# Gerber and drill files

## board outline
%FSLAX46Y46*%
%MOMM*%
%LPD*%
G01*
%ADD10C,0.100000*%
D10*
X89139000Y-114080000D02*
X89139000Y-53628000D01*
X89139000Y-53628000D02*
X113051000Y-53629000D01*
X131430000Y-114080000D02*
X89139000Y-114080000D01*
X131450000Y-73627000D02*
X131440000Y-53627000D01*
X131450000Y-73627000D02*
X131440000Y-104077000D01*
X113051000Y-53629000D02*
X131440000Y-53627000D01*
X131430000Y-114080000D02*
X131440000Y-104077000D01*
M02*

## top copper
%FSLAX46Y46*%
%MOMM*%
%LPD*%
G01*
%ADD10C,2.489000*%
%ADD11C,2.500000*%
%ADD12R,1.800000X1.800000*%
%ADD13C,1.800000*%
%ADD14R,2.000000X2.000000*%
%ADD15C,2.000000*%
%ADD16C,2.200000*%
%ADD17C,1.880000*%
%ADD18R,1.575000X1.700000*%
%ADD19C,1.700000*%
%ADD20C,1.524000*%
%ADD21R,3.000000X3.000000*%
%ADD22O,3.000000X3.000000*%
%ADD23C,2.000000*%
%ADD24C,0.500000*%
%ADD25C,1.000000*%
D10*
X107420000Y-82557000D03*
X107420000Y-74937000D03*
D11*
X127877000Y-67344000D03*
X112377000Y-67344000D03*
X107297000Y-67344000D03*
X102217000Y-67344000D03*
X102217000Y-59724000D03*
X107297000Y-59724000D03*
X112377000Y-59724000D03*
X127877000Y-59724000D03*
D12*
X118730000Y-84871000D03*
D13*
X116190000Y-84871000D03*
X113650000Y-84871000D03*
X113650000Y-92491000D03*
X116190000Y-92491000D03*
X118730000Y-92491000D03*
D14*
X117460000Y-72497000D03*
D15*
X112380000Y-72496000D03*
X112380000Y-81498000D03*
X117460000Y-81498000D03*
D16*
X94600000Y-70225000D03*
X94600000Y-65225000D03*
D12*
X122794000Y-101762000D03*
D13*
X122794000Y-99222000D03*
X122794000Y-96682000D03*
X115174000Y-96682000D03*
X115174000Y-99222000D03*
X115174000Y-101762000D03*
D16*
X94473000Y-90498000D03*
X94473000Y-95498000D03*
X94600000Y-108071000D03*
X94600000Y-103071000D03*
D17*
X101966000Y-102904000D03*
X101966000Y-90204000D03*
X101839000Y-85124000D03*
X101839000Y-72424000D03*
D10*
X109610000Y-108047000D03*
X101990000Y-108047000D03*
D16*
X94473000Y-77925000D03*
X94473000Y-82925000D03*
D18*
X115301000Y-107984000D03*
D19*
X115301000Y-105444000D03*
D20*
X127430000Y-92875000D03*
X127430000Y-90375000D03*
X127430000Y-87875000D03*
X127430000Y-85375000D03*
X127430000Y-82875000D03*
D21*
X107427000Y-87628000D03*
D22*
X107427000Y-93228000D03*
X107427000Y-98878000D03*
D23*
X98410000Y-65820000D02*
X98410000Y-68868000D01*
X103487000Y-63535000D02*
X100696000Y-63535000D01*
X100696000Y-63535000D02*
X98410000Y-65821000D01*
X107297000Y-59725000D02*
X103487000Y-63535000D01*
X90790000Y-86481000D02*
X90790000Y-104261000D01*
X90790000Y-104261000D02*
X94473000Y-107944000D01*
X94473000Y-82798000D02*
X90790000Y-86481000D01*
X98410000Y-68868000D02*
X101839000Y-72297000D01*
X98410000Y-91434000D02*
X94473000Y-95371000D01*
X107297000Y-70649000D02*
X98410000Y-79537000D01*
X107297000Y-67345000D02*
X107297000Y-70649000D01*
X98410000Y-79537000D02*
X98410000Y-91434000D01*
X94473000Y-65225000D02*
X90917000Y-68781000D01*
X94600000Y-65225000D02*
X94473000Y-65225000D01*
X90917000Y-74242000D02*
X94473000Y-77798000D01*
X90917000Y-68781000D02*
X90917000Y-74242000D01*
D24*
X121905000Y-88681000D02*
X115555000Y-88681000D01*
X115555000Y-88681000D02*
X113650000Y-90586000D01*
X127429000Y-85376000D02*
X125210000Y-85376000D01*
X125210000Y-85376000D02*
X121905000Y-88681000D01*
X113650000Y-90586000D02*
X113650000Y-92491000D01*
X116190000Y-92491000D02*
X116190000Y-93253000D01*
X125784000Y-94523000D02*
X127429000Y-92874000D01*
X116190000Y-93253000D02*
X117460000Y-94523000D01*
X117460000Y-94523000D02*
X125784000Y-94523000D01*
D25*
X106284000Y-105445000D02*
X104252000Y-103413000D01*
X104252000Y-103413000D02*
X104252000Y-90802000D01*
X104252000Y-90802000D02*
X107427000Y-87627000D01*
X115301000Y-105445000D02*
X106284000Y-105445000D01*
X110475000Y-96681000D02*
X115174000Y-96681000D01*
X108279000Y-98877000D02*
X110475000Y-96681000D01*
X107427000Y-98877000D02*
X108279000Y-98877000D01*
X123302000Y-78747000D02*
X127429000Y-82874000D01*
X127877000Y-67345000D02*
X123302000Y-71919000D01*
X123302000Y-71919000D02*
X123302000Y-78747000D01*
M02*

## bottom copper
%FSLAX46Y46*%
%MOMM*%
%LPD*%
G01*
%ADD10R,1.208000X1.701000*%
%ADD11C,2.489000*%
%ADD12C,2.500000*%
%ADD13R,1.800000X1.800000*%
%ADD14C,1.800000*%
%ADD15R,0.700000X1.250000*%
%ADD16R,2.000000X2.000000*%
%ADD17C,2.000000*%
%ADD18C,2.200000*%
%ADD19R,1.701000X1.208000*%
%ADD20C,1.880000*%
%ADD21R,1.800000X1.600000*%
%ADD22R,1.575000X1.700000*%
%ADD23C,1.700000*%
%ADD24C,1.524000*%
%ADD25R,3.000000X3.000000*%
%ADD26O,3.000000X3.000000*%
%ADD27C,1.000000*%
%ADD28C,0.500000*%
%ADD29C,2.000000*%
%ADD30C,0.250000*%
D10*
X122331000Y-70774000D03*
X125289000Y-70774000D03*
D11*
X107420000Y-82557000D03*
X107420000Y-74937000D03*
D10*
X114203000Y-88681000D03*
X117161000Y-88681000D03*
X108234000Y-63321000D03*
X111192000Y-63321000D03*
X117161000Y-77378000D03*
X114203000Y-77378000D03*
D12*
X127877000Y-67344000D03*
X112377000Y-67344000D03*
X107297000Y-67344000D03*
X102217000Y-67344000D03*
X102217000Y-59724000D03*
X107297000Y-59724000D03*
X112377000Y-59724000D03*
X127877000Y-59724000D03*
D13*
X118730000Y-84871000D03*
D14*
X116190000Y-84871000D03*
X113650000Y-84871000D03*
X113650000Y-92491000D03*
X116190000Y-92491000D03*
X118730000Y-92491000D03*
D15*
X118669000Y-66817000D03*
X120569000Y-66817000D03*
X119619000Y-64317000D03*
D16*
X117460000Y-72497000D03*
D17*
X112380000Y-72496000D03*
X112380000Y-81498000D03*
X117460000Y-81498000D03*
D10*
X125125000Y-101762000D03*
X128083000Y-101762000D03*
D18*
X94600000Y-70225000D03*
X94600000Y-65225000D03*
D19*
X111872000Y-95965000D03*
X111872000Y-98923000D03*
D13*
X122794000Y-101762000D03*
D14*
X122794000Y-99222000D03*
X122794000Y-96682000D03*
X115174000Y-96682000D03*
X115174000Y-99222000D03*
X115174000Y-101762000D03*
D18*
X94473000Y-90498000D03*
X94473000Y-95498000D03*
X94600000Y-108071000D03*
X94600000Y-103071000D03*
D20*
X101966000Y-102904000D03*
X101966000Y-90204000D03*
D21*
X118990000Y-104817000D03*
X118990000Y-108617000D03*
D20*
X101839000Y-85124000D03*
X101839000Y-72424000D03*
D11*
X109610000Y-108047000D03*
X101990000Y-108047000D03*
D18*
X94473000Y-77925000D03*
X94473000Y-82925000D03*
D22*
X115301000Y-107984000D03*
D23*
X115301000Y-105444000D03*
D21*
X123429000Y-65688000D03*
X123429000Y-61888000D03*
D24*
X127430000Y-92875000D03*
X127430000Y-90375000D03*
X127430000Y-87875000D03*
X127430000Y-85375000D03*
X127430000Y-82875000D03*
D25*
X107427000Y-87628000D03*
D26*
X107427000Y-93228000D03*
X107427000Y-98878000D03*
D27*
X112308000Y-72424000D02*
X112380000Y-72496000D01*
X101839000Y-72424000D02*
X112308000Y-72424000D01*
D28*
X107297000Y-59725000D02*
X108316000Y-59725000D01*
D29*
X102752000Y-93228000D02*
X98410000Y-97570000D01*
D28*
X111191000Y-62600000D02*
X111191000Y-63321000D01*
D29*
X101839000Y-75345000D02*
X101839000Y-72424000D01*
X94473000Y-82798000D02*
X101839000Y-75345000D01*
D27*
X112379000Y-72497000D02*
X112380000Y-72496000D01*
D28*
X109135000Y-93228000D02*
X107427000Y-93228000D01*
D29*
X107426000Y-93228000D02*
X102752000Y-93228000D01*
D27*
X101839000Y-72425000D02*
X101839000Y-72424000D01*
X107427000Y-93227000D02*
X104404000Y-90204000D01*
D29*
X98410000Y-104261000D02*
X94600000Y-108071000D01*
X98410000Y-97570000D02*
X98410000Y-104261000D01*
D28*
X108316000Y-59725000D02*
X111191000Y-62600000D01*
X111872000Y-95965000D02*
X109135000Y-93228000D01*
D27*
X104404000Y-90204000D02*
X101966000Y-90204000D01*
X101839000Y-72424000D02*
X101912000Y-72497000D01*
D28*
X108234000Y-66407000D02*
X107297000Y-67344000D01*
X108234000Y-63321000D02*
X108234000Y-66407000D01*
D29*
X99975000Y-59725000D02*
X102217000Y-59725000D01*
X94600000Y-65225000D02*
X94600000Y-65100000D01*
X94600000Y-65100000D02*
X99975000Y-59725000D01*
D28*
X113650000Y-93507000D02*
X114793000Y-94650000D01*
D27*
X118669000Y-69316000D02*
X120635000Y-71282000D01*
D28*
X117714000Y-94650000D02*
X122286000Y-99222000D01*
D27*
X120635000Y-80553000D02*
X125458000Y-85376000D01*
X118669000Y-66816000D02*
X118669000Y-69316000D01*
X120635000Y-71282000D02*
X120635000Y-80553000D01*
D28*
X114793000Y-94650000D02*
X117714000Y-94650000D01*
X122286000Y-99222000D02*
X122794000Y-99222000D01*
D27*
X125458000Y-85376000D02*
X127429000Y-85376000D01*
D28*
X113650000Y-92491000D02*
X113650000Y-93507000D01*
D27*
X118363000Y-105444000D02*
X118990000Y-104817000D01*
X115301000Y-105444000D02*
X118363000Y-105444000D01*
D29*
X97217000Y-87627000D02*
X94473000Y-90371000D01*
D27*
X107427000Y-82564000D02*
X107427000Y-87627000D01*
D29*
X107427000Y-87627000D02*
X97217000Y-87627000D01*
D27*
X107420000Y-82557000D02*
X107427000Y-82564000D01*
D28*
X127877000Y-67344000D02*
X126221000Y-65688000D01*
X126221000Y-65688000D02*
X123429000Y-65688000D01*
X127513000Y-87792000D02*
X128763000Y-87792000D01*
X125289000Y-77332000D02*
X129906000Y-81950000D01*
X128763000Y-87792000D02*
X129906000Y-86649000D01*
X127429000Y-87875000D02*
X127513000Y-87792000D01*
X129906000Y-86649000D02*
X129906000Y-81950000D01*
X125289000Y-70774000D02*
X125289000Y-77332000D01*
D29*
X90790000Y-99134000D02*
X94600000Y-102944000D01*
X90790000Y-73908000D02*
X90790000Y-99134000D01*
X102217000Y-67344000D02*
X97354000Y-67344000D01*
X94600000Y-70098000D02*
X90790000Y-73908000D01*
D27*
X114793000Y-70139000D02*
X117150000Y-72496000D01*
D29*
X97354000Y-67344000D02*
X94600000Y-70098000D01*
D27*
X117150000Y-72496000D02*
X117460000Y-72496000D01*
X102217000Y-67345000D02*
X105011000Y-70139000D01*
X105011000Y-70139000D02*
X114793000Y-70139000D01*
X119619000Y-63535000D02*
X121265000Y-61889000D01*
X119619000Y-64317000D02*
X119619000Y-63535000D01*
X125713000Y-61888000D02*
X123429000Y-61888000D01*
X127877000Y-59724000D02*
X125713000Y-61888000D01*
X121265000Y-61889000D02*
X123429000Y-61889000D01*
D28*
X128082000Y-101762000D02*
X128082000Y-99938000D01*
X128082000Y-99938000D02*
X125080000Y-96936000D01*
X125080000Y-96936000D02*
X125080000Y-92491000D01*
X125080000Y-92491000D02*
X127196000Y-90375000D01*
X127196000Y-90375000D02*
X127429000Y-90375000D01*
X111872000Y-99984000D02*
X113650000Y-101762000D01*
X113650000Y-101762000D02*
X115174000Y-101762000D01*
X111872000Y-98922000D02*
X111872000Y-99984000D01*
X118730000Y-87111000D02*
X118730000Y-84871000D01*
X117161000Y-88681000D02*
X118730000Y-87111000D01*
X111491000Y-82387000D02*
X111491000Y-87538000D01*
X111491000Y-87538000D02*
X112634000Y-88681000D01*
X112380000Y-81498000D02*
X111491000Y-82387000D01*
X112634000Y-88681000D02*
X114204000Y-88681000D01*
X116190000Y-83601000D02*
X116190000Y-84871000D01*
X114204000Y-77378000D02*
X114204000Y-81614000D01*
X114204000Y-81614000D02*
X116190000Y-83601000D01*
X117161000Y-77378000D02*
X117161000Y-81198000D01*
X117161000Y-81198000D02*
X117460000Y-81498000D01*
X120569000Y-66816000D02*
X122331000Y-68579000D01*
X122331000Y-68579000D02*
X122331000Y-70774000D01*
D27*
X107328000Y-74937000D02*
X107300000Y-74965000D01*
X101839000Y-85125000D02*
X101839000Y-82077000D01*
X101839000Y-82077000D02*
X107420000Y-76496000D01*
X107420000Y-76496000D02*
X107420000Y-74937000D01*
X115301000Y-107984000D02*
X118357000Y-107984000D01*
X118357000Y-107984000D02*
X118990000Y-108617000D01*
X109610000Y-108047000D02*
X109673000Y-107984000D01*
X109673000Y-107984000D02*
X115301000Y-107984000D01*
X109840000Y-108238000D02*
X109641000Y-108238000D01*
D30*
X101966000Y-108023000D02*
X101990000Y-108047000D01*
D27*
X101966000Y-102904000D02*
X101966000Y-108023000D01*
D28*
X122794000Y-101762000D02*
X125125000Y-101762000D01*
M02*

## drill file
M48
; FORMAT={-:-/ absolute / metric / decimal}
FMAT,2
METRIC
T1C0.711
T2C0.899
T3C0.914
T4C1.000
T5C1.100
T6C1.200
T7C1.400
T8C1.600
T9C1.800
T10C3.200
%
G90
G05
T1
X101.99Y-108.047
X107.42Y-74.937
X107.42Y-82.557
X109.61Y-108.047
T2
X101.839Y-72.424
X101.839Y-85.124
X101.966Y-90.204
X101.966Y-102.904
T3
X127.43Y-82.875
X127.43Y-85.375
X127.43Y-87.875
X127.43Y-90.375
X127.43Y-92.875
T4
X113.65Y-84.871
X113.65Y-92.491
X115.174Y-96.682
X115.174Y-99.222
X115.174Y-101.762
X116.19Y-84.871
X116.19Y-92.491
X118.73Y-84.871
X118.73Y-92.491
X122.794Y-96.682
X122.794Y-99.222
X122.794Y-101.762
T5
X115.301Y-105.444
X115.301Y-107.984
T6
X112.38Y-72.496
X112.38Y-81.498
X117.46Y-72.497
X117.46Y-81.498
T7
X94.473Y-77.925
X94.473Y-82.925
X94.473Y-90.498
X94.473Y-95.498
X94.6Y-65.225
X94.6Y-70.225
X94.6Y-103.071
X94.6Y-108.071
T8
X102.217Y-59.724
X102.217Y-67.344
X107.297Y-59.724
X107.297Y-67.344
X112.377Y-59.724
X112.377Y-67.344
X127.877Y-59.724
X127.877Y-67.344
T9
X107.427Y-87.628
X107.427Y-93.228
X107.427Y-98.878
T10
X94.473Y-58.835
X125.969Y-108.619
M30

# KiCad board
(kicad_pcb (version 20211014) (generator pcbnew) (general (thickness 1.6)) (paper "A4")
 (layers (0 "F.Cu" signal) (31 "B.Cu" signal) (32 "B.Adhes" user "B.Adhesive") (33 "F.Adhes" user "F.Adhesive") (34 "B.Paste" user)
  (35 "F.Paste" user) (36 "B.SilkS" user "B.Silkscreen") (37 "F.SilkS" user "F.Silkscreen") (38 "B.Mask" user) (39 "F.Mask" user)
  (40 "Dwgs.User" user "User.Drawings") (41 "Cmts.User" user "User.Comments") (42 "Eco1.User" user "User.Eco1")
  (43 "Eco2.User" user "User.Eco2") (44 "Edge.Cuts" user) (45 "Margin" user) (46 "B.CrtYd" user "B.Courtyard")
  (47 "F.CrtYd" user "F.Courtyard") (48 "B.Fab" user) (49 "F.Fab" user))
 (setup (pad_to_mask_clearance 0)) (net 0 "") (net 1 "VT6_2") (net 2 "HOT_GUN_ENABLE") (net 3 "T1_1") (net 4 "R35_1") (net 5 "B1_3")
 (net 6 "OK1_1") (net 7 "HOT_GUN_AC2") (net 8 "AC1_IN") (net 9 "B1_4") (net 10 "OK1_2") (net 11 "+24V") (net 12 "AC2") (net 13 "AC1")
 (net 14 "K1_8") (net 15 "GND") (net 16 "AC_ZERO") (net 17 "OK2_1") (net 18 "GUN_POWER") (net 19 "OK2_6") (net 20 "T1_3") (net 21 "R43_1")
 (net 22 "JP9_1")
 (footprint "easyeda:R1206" (layer "F.Cu") (at 123.81 70.774 180)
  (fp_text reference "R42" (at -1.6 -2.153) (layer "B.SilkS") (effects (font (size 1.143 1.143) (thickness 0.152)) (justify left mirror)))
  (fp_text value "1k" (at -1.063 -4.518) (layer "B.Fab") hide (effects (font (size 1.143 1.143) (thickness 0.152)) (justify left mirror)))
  (pad "1" smd rect locked (at 1.479 0 180) (size 1.208 1.701) (layers "B.Cu" "B.Paste" "B.Mask") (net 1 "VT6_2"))
  (pad "2" smd rect locked (at -1.479 0 180) (size 1.208 1.701) (layers "B.Cu" "B.Paste" "B.Mask") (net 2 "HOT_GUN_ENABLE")))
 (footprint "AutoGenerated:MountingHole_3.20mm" (layer "F.Cu") (at 125.969 108.619)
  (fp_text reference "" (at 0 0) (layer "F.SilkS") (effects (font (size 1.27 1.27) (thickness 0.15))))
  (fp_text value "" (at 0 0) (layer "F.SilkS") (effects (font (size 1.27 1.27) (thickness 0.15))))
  (pad "" np_thru_hole circle locked (at 0 0) (size 3.2 3.2) (drill 3.2) (layers *.Cu *.Mask)))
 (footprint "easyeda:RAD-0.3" (layer "F.Cu") (at 107.42 78.747 -90)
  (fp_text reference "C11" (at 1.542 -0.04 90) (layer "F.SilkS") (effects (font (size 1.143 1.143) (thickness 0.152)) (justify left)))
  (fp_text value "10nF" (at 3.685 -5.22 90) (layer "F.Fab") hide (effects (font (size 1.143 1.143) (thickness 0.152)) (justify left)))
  (pad "1" thru_hole circle locked (at 3.81 0 90) (size 2.489 2.489) (drill 0.711) (layers *.Cu *.Paste *.Mask) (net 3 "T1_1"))
  (pad "2" thru_hole circle locked (at -3.81 0 90) (size 2.489 2.489) (drill 0.711) (layers *.Cu *.Paste *.Mask) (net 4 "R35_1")))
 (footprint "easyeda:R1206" (layer "F.Cu") (at 115.682 88.681 180)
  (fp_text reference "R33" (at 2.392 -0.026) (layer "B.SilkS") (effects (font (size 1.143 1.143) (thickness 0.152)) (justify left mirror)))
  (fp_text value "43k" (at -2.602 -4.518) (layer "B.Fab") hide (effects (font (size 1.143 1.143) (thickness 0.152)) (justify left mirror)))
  (pad "1" smd rect locked (at 1.479 0 180) (size 1.208 1.701) (layers "B.Cu" "B.Paste" "B.Mask") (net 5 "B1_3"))
  (pad "2" smd rect locked (at -1.479 0 180) (size 1.208 1.701) (layers "B.Cu" "B.Paste" "B.Mask") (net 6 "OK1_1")))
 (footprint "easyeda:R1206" (layer "F.Cu") (at 109.713 63.321 180)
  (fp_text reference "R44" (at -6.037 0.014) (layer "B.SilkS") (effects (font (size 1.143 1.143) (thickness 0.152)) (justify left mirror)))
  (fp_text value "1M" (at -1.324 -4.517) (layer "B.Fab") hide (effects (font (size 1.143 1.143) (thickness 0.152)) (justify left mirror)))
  (pad "1" smd rect locked (at 1.479 0 180) (size 1.208 1.701) (layers "B.Cu" "B.Paste" "B.Mask") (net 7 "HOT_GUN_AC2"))
  (pad "2" smd rect locked (at -1.479 0 180) (size 1.208 1.701) (layers "B.Cu" "B.Paste" "B.Mask") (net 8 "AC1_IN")))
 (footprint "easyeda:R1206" (layer "F.Cu") (at 115.682 77.378)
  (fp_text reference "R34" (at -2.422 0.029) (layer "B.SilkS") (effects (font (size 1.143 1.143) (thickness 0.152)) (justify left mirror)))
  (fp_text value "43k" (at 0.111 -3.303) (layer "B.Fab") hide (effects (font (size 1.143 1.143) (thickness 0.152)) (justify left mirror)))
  (pad "1" smd rect locked (at 1.479 0) (size 1.208 1.701) (layers "B.Cu" "B.Paste" "B.Mask") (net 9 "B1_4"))
  (pad "2" smd rect locked (at -1.479 0) (size 1.208 1.701) (layers "B.Cu" "B.Paste" "B.Mask") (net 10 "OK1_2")))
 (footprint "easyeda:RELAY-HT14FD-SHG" (layer "F.Cu") (at 115.047 63.534 180)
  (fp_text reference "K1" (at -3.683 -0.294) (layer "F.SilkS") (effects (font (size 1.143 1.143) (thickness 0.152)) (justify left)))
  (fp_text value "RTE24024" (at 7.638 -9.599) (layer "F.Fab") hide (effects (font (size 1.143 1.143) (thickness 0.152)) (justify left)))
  (pad "1" thru_hole circle locked (at -12.83 -3.81 180) (size 2.5 2.5) (drill 1.6) (layers *.Cu *.Paste *.Mask) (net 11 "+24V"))
  (pad "2" thru_hole circle locked (at 2.67 -3.81 180) (size 2.5 2.5) (drill 1.6) (layers *.Cu *.Paste *.Mask))
  (pad "3" thru_hole circle locked (at 7.75 -3.81 180) (size 2.5 2.5) (drill 1.6) (layers *.Cu *.Paste *.Mask) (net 7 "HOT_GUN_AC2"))
  (pad "4" thru_hole circle locked (at 12.83 -3.81 180) (size 2.5 2.5) (drill 1.6) (layers *.Cu *.Paste *.Mask) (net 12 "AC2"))
  (pad "5" thru_hole circle locked (at 12.83 3.81 180) (size 2.5 2.5) (drill 1.6) (layers *.Cu *.Paste *.Mask) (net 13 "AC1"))
  (pad "6" thru_hole circle locked (at 7.75 3.81 180) (size 2.5 2.5) (drill 1.6) (layers *.Cu *.Paste *.Mask) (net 8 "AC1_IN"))
  (pad "7" thru_hole circle locked (at 2.67 3.81 180) (size 2.5 2.5) (drill 1.6) (layers *.Cu *.Paste *.Mask))
  (pad "8" thru_hole circle locked (at -12.83 3.81 180) (size 2.5 2.5) (drill 1.6) (layers *.Cu *.Paste *.Mask) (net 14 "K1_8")))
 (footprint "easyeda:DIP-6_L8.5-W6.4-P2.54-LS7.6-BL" (layer "F.Cu") (at 116.19 88.681 180)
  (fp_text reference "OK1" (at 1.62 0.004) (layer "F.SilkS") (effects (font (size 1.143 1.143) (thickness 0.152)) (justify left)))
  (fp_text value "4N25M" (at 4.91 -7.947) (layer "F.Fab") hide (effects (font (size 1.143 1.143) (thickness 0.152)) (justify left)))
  (pad "1" thru_hole rect locked (at -2.54 3.81 270) (size 1.8 1.8) (drill 1) (layers *.Cu *.Paste *.Mask) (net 6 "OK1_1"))
  (pad "2" thru_hole circle locked (at 0 3.81 270) (size 1.8 1.8) (drill 1) (layers *.Cu *.Paste *.Mask) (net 10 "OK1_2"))
  (pad "3" thru_hole circle locked (at 2.54 3.81 270) (size 1.8 1.8) (drill 1) (layers *.Cu *.Paste *.Mask))
  (pad "4" thru_hole circle locked (at 2.54 -3.81 270) (size 1.8 1.8) (drill 1) (layers *.Cu *.Paste *.Mask) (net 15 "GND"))
  (pad "5" thru_hole circle locked (at 0 -3.81 270) (size 1.8 1.8) (drill 1) (layers *.Cu *.Paste *.Mask) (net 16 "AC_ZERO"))
  (pad "6" thru_hole circle locked (at -2.54 -3.81 270) (size 1.8 1.8) (drill 1) (layers *.Cu *.Paste *.Mask)))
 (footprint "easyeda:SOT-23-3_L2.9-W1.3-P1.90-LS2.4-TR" (layer "F.Cu") (at 119.619 65.567 90)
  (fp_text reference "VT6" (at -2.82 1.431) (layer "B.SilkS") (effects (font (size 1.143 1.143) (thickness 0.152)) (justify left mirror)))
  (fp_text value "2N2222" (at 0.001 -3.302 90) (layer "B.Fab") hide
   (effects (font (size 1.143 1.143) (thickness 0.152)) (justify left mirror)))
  (pad "1" smd rect locked (at -1.25 -0.95 180) (size 0.7 1.25) (layers "B.Cu" "B.Paste" "B.Mask") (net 15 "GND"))
  (pad "2" smd rect locked (at -1.25 0.95 180) (size 0.7 1.25) (layers "B.Cu" "B.Paste" "B.Mask") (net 1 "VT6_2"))
  (pad "3" smd rect locked (at 1.25 0 180) (size 0.7 1.25) (layers "B.Cu" "B.Paste" "B.Mask") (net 14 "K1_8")))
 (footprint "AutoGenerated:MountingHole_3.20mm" (layer "F.Cu") (at 94.473 58.835)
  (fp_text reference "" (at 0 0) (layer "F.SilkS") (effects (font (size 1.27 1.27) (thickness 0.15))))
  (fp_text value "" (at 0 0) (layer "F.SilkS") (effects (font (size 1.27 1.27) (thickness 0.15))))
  (pad "" np_thru_hole circle locked (at 0 0) (size 3.2 3.2) (drill 3.2) (layers *.Cu *.Mask)))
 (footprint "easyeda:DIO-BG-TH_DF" (layer "F.Cu") (at 114.92 76.997 -90)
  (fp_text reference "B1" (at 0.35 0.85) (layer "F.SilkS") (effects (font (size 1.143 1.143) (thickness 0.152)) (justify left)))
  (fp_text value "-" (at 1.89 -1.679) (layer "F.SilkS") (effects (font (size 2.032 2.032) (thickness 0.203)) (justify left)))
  (pad "1" thru_hole rect locked (at -4.5 -2.54 270) (size 2 2) (drill 1.2) (layers *.Cu *.Paste *.Mask) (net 12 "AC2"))
  (pad "2" thru_hole circle locked (at -4.501 2.54 270) (size 2 2) (drill 1.2) (layers *.Cu *.Paste *.Mask) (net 8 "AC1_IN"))
  (pad "3" thru_hole circle locked (at 4.501 2.54 270) (size 2 2) (drill 1.2) (layers *.Cu *.Paste *.Mask) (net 5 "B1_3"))
  (pad "4" thru_hole circle locked (at 4.501 -2.54 270) (size 2 2) (drill 1.2) (layers *.Cu *.Paste *.Mask) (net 9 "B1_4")))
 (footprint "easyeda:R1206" (layer "F.Cu") (at 126.604 101.762 180)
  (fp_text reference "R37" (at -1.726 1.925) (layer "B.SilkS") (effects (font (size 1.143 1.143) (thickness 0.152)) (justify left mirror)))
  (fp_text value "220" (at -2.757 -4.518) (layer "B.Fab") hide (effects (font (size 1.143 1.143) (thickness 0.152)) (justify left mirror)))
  (pad "1" smd rect locked (at 1.479 0 180) (size 1.208 1.701) (layers "B.Cu" "B.Paste" "B.Mask") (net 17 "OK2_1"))
  (pad "2" smd rect locked (at -1.479 0 180) (size 1.208 1.701) (layers "B.Cu" "B.Paste" "B.Mask") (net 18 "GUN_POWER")))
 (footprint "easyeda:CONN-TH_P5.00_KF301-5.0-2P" (layer "F.Cu") (at 94.6 67.725 90)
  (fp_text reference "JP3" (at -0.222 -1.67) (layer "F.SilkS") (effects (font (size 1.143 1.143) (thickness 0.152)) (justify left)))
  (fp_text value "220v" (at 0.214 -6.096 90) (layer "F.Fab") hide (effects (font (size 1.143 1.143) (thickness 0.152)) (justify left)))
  (pad "1" thru_hole circle locked (at -2.5 0 90) (size 2.2 2.2) (drill 1.4) (layers *.Cu *.Paste *.Mask) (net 12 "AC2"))
  (pad "2" thru_hole circle locked (at 2.5 0 90) (size 2.2 2.2) (drill 1.4) (layers *.Cu *.Paste *.Mask) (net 13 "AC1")))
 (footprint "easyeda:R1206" (layer "F.Cu") (at 111.872 97.444 90)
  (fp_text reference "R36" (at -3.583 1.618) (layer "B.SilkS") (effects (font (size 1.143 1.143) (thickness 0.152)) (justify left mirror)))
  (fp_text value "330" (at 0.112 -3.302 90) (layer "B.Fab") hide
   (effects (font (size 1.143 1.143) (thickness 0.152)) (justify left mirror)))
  (pad "1" smd rect locked (at 1.479 0 90) (size 1.208 1.701) (layers "B.Cu" "B.Paste" "B.Mask") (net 8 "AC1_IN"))
  (pad "2" smd rect locked (at -1.479 0 90) (size 1.208 1.701) (layers "B.Cu" "B.Paste" "B.Mask") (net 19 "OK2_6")))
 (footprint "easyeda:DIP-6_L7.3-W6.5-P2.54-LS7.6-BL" (layer "F.Cu") (at 118.984 99.222 90)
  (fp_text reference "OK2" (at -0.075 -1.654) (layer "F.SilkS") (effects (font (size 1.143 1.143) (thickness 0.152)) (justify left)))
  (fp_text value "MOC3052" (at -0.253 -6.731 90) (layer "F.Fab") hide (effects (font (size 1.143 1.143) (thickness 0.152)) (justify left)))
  (pad "1" thru_hole rect locked (at -2.54 3.81 180) (size 1.8 1.8) (drill 1) (layers *.Cu *.Paste *.Mask) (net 17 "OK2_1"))
  (pad "2" thru_hole circle locked (at 0 3.81 180) (size 1.8 1.8) (drill 1) (layers *.Cu *.Paste *.Mask) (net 15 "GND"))
  (pad "3" thru_hole circle locked (at 2.54 3.81 180) (size 1.8 1.8) (drill 1) (layers *.Cu *.Paste *.Mask))
  (pad "4" thru_hole circle locked (at 2.54 -3.81 180) (size 1.8 1.8) (drill 1) (layers *.Cu *.Paste *.Mask) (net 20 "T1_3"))
  (pad "5" thru_hole circle locked (at 0 -3.81 180) (size 1.8 1.8) (drill 1) (layers *.Cu *.Paste *.Mask))
  (pad "6" thru_hole circle locked (at -2.54 -3.81 180) (size 1.8 1.8) (drill 1) (layers *.Cu *.Paste *.Mask) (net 19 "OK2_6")))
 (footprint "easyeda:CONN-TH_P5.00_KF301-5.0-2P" (layer "F.Cu") (at 94.473 92.998 -90)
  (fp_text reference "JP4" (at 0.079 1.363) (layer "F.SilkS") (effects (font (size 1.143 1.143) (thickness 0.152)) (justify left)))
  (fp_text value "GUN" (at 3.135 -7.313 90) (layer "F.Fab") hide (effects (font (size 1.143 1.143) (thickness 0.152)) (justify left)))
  (pad "1" thru_hole circle locked (at -2.5 0 270) (size 2.2 2.2) (drill 1.4) (layers *.Cu *.Paste *.Mask) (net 3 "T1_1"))
  (pad "2" thru_hole circle locked (at 2.5 0 270) (size 2.2 2.2) (drill 1.4) (layers *.Cu *.Paste *.Mask) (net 7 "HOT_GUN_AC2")))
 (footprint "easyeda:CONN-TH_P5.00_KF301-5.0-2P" (layer "F.Cu") (at 94.6 105.571 90)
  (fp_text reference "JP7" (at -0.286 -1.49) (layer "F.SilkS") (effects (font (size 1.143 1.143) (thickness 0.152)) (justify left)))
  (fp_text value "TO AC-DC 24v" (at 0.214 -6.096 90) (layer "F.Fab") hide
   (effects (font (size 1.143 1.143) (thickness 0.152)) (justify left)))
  (pad "1" thru_hole circle locked (at -2.5 0 90) (size 2.2 2.2) (drill 1.4) (layers *.Cu *.Paste *.Mask) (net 8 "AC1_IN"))
  (pad "2" thru_hole circle locked (at 2.5 0 90) (size 2.2 2.2) (drill 1.4) (layers *.Cu *.Paste *.Mask) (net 12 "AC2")))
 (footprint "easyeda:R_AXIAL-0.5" (layer "F.Cu") (at 101.966 96.554 90)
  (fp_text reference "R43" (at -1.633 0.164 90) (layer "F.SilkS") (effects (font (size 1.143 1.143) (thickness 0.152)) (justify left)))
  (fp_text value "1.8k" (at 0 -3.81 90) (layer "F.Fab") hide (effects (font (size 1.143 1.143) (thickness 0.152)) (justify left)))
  (pad "1" thru_hole circle locked (at -6.35 0 90) (size 1.88 1.88) (drill 0.899) (layers *.Cu *.Paste *.Mask) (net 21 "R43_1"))
  (pad "2" thru_hole circle locked (at 6.35 0 90) (size 1.88 1.88) (drill 0.899) (layers *.Cu *.Paste *.Mask) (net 8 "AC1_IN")))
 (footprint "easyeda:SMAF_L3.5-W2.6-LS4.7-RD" (layer "F.Cu") (at 118.99 106.717 90)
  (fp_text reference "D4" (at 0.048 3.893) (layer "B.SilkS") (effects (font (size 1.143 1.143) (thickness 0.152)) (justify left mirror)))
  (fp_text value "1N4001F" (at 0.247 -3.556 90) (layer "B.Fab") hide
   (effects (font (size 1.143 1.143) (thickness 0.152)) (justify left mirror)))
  (pad "1" smd rect locked (at 1.9 0 270) (size 1.6 1.8) (layers "B.Cu" "B.Paste" "B.Mask") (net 3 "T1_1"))
  (pad "2" smd rect locked (at -1.9 0 270) (size 1.6 1.8) (layers "B.Cu" "B.Paste" "B.Mask") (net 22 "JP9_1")))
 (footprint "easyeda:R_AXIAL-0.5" (layer "F.Cu") (at 101.839 78.774 90)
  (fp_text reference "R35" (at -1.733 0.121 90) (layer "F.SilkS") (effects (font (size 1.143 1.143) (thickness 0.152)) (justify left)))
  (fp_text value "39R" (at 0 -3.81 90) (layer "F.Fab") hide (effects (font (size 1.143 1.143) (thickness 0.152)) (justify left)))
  (pad "1" thru_hole circle locked (at -6.35 0 90) (size 1.88 1.88) (drill 0.899) (layers *.Cu *.Paste *.Mask) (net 4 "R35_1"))
  (pad "2" thru_hole circle locked (at 6.35 0 90) (size 1.88 1.88) (drill 0.899) (layers *.Cu *.Paste *.Mask) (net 8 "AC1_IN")))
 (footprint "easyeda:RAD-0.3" (layer "F.Cu") (at 105.8 108.047)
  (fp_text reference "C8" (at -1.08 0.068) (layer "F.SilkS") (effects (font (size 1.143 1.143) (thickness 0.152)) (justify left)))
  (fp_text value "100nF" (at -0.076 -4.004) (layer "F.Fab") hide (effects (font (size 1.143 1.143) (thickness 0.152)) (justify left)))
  (pad "1" thru_hole circle locked (at 3.81 0 180) (size 2.489 2.489) (drill 0.711) (layers *.Cu *.Paste *.Mask) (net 22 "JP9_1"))
  (pad "2" thru_hole circle locked (at -3.81 0 180) (size 2.489 2.489) (drill 0.711) (layers *.Cu *.Paste *.Mask) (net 21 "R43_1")))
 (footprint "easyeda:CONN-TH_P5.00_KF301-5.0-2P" (layer "F.Cu") (at 94.473 80.425 -90)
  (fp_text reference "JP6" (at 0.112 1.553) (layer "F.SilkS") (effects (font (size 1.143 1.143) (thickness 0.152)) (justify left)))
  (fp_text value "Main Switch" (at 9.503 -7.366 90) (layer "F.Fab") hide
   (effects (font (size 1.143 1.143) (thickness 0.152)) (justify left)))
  (pad "1" thru_hole circle locked (at -2.5 0 270) (size 2.2 2.2) (drill 1.4) (layers *.Cu *.Paste *.Mask) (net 13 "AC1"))
  (pad "2" thru_hole circle locked (at 2.5 0 270) (size 2.2 2.2) (drill 1.4) (layers *.Cu *.Paste *.Mask) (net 8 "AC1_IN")))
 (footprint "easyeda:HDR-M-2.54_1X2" (layer "F.Cu") (at 115.301 106.714 90)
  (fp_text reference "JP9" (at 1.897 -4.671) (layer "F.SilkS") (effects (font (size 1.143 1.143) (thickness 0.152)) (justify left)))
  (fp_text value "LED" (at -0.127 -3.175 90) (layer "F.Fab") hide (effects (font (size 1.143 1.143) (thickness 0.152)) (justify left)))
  (pad "1" thru_hole rect locked (at -1.27 0 90) (size 1.7 1.575) (drill 1.1) (layers *.Cu *.Paste *.Mask) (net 22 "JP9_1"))
  (pad "2" thru_hole circle locked (at 1.27 0 90) (size 1.7 1.7) (drill 1.1) (layers *.Cu *.Paste *.Mask) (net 3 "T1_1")))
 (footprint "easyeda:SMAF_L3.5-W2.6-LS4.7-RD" (layer "F.Cu") (at 123.429 63.788 -90)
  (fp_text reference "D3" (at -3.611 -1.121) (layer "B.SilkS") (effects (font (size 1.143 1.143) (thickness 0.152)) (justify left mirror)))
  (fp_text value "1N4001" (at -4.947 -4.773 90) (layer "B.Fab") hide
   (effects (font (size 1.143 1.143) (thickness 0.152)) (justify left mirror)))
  (pad "1" smd rect locked (at 1.9 0 90) (size 1.6 1.8) (layers "B.Cu" "B.Paste" "B.Mask") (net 11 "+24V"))
  (pad "2" smd rect locked (at -1.9 0 90) (size 1.6 1.8) (layers "B.Cu" "B.Paste" "B.Mask") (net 14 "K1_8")))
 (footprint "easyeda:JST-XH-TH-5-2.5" (layer "F.Cu") (at 125.08 80.425 -90)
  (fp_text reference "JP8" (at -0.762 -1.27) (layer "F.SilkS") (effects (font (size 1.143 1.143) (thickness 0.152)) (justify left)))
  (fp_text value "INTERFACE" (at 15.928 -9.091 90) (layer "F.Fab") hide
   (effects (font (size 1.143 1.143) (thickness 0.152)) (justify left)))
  (pad "1" thru_hole circle locked (at 12.45 -2.35 270) (size 1.524 1.524) (drill 0.914) (layers *.Cu *.Paste *.Mask) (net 16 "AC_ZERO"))
  (pad "2" thru_hole circle locked (at 9.95 -2.35 270) (size 1.524 1.524) (drill 0.914) (layers *.Cu *.Paste *.Mask) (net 18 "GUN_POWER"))
  (pad "3" thru_hole circle locked (at 7.45 -2.35 270) (size 1.524 1.524) (drill 0.914) (layers *.Cu *.Paste *.Mask)
   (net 2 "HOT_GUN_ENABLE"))
  (pad "4" thru_hole circle locked (at 4.95 -2.35 270) (size 1.524 1.524) (drill 0.914) (layers *.Cu *.Paste *.Mask) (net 15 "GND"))
  (pad "5" thru_hole circle locked (at 2.45 -2.35 270) (size 1.524 1.524) (drill 0.914) (layers *.Cu *.Paste *.Mask) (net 11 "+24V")))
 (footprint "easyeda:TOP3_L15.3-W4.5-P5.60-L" (layer "F.Cu") (at 107.427 93.253 -90)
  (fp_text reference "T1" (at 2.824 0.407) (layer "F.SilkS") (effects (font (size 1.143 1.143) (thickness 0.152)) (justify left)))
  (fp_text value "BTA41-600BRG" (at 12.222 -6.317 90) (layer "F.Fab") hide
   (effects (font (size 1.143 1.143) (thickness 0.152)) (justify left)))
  (pad "1" thru_hole rect locked (at -5.625 0 270) (size 3 3) (drill 1.8) (layers *.Cu *.Paste *.Mask) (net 3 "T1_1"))
  (pad "2" thru_hole oval locked (at -0.025 0 270) (size 3 3) (drill 1.8) (layers *.Cu *.Paste *.Mask) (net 8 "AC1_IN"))
  (pad "3" thru_hole oval locked (at 5.625 0 270) (size 3 3) (drill 1.8) (layers *.Cu *.Paste *.Mask) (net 20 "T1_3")))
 (gr_line (start 89.139 114.08) (end 89.139 53.628) (layer "Edge.Cuts") (width 0.1))
 (gr_line (start 89.139 53.628) (end 113.051 53.629) (layer "Edge.Cuts") (width 0.1))
 (gr_line (start 131.43 114.08) (end 89.139 114.08) (layer "Edge.Cuts") (width 0.1))
 (gr_line (start 131.45 73.627) (end 131.44 53.627) (layer "Edge.Cuts") (width 0.1))
 (gr_line (start 131.45 73.627) (end 131.44 104.077) (layer "Edge.Cuts") (width 0.1))
 (gr_line (start 113.051 53.629) (end 131.44 53.627) (layer "Edge.Cuts") (width 0.1))
 (gr_line (start 131.43 114.08) (end 131.44 104.077) (layer "Edge.Cuts") (width 0.1))
 (segment (start 98.41 65.82) (end 98.41 68.868) (width 2) (layer "F.Cu") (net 8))
 (segment (start 103.487 63.535) (end 100.696 63.535) (width 2) (layer "F.Cu") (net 8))
 (segment (start 100.696 63.535) (end 98.41 65.821) (width 2) (layer "F.Cu") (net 8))
 (segment (start 107.297 59.725) (end 103.487 63.535) (width 2) (layer "F.Cu") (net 8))
 (segment (start 90.79 86.481) (end 90.79 104.261) (width 2) (layer "F.Cu") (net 8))
 (segment (start 90.79 104.261) (end 94.473 107.944) (width 2) (layer "F.Cu") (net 8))
 (segment (start 94.473 82.798) (end 90.79 86.481) (width 2) (layer "F.Cu") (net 8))
 (segment (start 98.41 68.868) (end 101.839 72.297) (width 2) (layer "F.Cu") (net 8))
 (segment (start 112.308 72.424) (end 112.38 72.496) (width 1) (layer "B.Cu") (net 8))
 (segment (start 101.839 72.424) (end 112.308 72.424) (width 1) (layer "B.Cu") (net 8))
 (segment (start 107.297 59.725) (end 108.316 59.725) (width 0.5) (layer "B.Cu") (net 8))
 (segment (start 102.752 93.228) (end 98.41 97.57) (width 2) (layer "B.Cu") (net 8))
 (segment (start 111.191 62.6) (end 111.191 63.321) (width 0.5) (layer "B.Cu") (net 8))
 (segment (start 101.839 75.345) (end 101.839 72.424) (width 2) (layer "B.Cu") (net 8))
 (segment (start 94.473 82.798) (end 101.839 75.345) (width 2) (layer "B.Cu") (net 8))
 (segment (start 112.379 72.497) (end 112.38 72.496) (width 1) (layer "B.Cu") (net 8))
 (segment (start 109.135 93.228) (end 107.427 93.228) (width 0.5) (layer "B.Cu") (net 8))
 (segment (start 107.426 93.228) (end 102.752 93.228) (width 2) (layer "B.Cu") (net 8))
 (segment (start 101.839 72.425) (end 101.839 72.424) (width 1) (layer "B.Cu") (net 8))
 (segment (start 107.427 93.227) (end 104.404 90.204) (width 1) (layer "B.Cu") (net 8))
 (segment (start 98.41 104.261) (end 94.6 108.071) (width 2) (layer "B.Cu") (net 8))
 (segment (start 98.41 97.57) (end 98.41 104.261) (width 2) (layer "B.Cu") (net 8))
 (segment (start 108.316 59.725) (end 111.191 62.6) (width 0.5) (layer "B.Cu") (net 8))
 (segment (start 111.872 95.965) (end 109.135 93.228) (width 0.5) (layer "B.Cu") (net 8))
 (segment (start 104.404 90.204) (end 101.966 90.204) (width 1) (layer "B.Cu") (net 8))
 (segment (start 101.839 72.424) (end 101.912 72.497) (width 1) (layer "B.Cu") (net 8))
 (segment (start 98.41 91.434) (end 94.473 95.371) (width 2) (layer "F.Cu") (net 7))
 (segment (start 107.297 70.649) (end 98.41 79.537) (width 2) (layer "F.Cu") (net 7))
 (segment (start 107.297 67.345) (end 107.297 70.649) (width 2) (layer "F.Cu") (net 7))
 (segment (start 98.41 79.537) (end 98.41 91.434) (width 2) (layer "F.Cu") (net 7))
 (segment (start 108.234 66.407) (end 107.297 67.344) (width 0.5) (layer "B.Cu") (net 7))
 (segment (start 108.234 63.321) (end 108.234 66.407) (width 0.5) (layer "B.Cu") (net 7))
 (segment (start 94.473 65.225) (end 90.917 68.781) (width 2) (layer "F.Cu") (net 13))
 (segment (start 94.6 65.225) (end 94.473 65.225) (width 2) (layer "F.Cu") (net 13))
 (segment (start 90.917 74.242) (end 94.473 77.798) (width 2) (layer "F.Cu") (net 13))
 (segment (start 90.917 68.781) (end 90.917 74.242) (width 2) (layer "F.Cu") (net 13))
 (segment (start 99.975 59.725) (end 102.217 59.725) (width 2) (layer "B.Cu") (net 13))
 (segment (start 94.6 65.225) (end 94.6 65.1) (width 2) (layer "B.Cu") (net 13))
 (segment (start 94.6 65.1) (end 99.975 59.725) (width 2) (layer "B.Cu") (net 13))
 (segment (start 121.905 88.681) (end 115.555 88.681) (width 0.5) (layer "F.Cu") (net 15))
 (segment (start 115.555 88.681) (end 113.65 90.586) (width 0.5) (layer "F.Cu") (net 15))
 (segment (start 127.429 85.376) (end 125.21 85.376) (width 0.5) (layer "F.Cu") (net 15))
 (segment (start 125.21 85.376) (end 121.905 88.681) (width 0.5) (layer "F.Cu") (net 15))
 (segment (start 113.65 90.586) (end 113.65 92.491) (width 0.5) (layer "F.Cu") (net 15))
 (segment (start 113.65 93.507) (end 114.793 94.65) (width 0.5) (layer "B.Cu") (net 15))
 (segment (start 118.669 69.316) (end 120.635 71.282) (width 1) (layer "B.Cu") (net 15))
 (segment (start 117.714 94.65) (end 122.286 99.222) (width 0.5) (layer "B.Cu") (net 15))
 (segment (start 120.635 80.553) (end 125.458 85.376) (width 1) (layer "B.Cu") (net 15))
 (segment (start 118.669 66.816) (end 118.669 69.316) (width 1) (layer "B.Cu") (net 15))
 (segment (start 120.635 71.282) (end 120.635 80.553) (width 1) (layer "B.Cu") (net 15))
 (segment (start 114.793 94.65) (end 117.714 94.65) (width 0.5) (layer "B.Cu") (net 15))
 (segment (start 122.286 99.222) (end 122.794 99.222) (width 0.5) (layer "B.Cu") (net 15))
 (segment (start 125.458 85.376) (end 127.429 85.376) (width 1) (layer "B.Cu") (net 15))
 (segment (start 113.65 92.491) (end 113.65 93.507) (width 0.5) (layer "B.Cu") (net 15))
 (segment (start 116.19 92.491) (end 116.19 93.253) (width 0.5) (layer "F.Cu") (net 16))
 (segment (start 125.784 94.523) (end 127.429 92.874) (width 0.5) (layer "F.Cu") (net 16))
 (segment (start 116.19 93.253) (end 117.46 94.523) (width 0.5) (layer "F.Cu") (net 16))
 (segment (start 117.46 94.523) (end 125.784 94.523) (width 0.5) (layer "F.Cu") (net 16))
 (segment (start 106.284 105.445) (end 104.252 103.413) (width 1) (layer "F.Cu") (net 3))
 (segment (start 104.252 103.413) (end 104.252 90.802) (width 1) (layer "F.Cu") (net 3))
 (segment (start 104.252 90.802) (end 107.427 87.627) (width 1) (layer "F.Cu") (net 3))
 (segment (start 115.301 105.445) (end 106.284 105.445) (width 1) (layer "F.Cu") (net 3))
 (segment (start 118.363 105.444) (end 118.99 104.817) (width 1) (layer "B.Cu") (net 3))
 (segment (start 115.301 105.444) (end 118.363 105.444) (width 1) (layer "B.Cu") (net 3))
 (segment (start 97.217 87.627) (end 94.473 90.371) (width 2) (layer "B.Cu") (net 3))
 (segment (start 107.427 82.564) (end 107.427 87.627) (width 1) (layer "B.Cu") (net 3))
 (segment (start 107.427 87.627) (end 97.217 87.627) (width 2) (layer "B.Cu") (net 3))
 (segment (start 107.42 82.557) (end 107.427 82.564) (width 1) (layer "B.Cu") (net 3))
 (segment (start 110.475 96.681) (end 115.174 96.681) (width 1) (layer "F.Cu") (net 20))
 (segment (start 108.279 98.877) (end 110.475 96.681) (width 1) (layer "F.Cu") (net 20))
 (segment (start 107.427 98.877) (end 108.279 98.877) (width 1) (layer "F.Cu") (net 20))
 (segment (start 123.302 78.747) (end 127.429 82.874) (width 1) (layer "F.Cu") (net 11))
 (segment (start 127.877 67.345) (end 123.302 71.919) (width 1) (layer "F.Cu") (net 11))
 (segment (start 123.302 71.919) (end 123.302 78.747) (width 1) (layer "F.Cu") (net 11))
 (segment (start 127.877 67.344) (end 126.221 65.688) (width 0.5) (layer "B.Cu") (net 11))
 (segment (start 126.221 65.688) (end 123.429 65.688) (width 0.5) (layer "B.Cu") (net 11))
 (segment (start 127.513 87.792) (end 128.763 87.792) (width 0.5) (layer "B.Cu") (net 2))
 (segment (start 125.289 77.332) (end 129.906 81.95) (width 0.5) (layer "B.Cu") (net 2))
 (segment (start 128.763 87.792) (end 129.906 86.649) (width 0.5) (layer "B.Cu") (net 2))
 (segment (start 127.429 87.875) (end 127.513 87.792) (width 0.5) (layer "B.Cu") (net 2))
 (segment (start 129.906 86.649) (end 129.906 81.95) (width 0.5) (layer "B.Cu") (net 2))
 (segment (start 125.289 70.774) (end 125.289 77.332) (width 0.5) (layer "B.Cu") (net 2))
 (segment (start 90.79 99.134) (end 94.6 102.944) (width 2) (layer "B.Cu") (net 12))
 (segment (start 90.79 73.908) (end 90.79 99.134) (width 2) (layer "B.Cu") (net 12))
 (segment (start 102.217 67.344) (end 97.354 67.344) (width 2) (layer "B.Cu") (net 12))
 (segment (start 94.6 70.098) (end 90.79 73.908) (width 2) (layer "B.Cu") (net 12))
 (segment (start 114.793 70.139) (end 117.15 72.496) (width 1) (layer "B.Cu") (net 12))
 (segment (start 97.354 67.344) (end 94.6 70.098) (width 2) (layer "B.Cu") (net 12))
 (segment (start 117.15 72.496) (end 117.46 72.496) (width 1) (layer "B.Cu") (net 12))
 (segment (start 102.217 67.345) (end 105.011 70.139) (width 1) (layer "B.Cu") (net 12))
 (segment (start 105.011 70.139) (end 114.793 70.139) (width 1) (layer "B.Cu") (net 12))
 (segment (start 119.619 63.535) (end 121.265 61.889) (width 1) (layer "B.Cu") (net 14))
 (segment (start 119.619 64.317) (end 119.619 63.535) (width 1) (layer "B.Cu") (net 14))
 (segment (start 125.713 61.888) (end 123.429 61.888) (width 1) (layer "B.Cu") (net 14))
 (segment (start 127.877 59.724) (end 125.713 61.888) (width 1) (layer "B.Cu") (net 14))
 (segment (start 121.265 61.889) (end 123.429 61.889) (width 1) (layer "B.Cu") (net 14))
 (segment (start 128.082 101.762) (end 128.082 99.938) (width 0.5) (layer "B.Cu") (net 18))
 (segment (start 128.082 99.938) (end 125.08 96.936) (width 0.5) (layer "B.Cu") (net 18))
 (segment (start 125.08 96.936) (end 125.08 92.491) (width 0.5) (layer "B.Cu") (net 18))
 (segment (start 125.08 92.491) (end 127.196 90.375) (width 0.5) (layer "B.Cu") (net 18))
 (segment (start 127.196 90.375) (end 127.429 90.375) (width 0.5) (layer "B.Cu") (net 18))
 (segment (start 111.872 99.984) (end 113.65 101.762) (width 0.5) (layer "B.Cu") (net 19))
 (segment (start 113.65 101.762) (end 115.174 101.762) (width 0.5) (layer "B.Cu") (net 19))
 (segment (start 111.872 98.922) (end 111.872 99.984) (width 0.5) (layer "B.Cu") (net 19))
 (segment (start 118.73 87.111) (end 118.73 84.871) (width 0.5) (layer "B.Cu") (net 6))
 (segment (start 117.161 88.681) (end 118.73 87.111) (width 0.5) (layer "B.Cu") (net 6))
 (segment (start 111.491 82.387) (end 111.491 87.538) (width 0.5) (layer "B.Cu") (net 5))
 (segment (start 111.491 87.538) (end 112.634 88.681) (width 0.5) (layer "B.Cu") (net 5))
 (segment (start 112.38 81.498) (end 111.491 82.387) (width 0.5) (layer "B.Cu") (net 5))
 (segment (start 112.634 88.681) (end 114.204 88.681) (width 0.5) (layer "B.Cu") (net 5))
 (segment (start 116.19 83.601) (end 116.19 84.871) (width 0.5) (layer "B.Cu") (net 10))
 (segment (start 114.204 77.378) (end 114.204 81.614) (width 0.5) (layer "B.Cu") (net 10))
 (segment (start 114.204 81.614) (end 116.19 83.601) (width 0.5) (layer "B.Cu") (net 10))
 (segment (start 117.161 77.378) (end 117.161 81.198) (width 0.5) (layer "B.Cu") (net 9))
 (segment (start 117.161 81.198) (end 117.46 81.498) (width 0.5) (layer "B.Cu") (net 9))
 (segment (start 120.569 66.816) (end 122.331 68.579) (width 0.5) (layer "B.Cu") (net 1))
 (segment (start 122.331 68.579) (end 122.331 70.774) (width 0.5) (layer "B.Cu") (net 1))
 (segment (start 107.328 74.937) (end 107.3 74.965) (width 1) (layer "B.Cu") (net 4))
 (segment (start 101.839 85.125) (end 101.839 82.077) (width 1) (layer "B.Cu") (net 4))
 (segment (start 101.839 82.077) (end 107.42 76.496) (width 1) (layer "B.Cu") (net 4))
 (segment (start 107.42 76.496) (end 107.42 74.937) (width 1) (layer "B.Cu") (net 4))
 (segment (start 115.301 107.984) (end 118.357 107.984) (width 1) (layer "B.Cu") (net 22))
 (segment (start 118.357 107.984) (end 118.99 108.617) (width 1) (layer "B.Cu") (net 22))
 (segment (start 109.61 108.047) (end 109.673 107.984) (width 1) (layer "B.Cu") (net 22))
 (segment (start 109.673 107.984) (end 115.301 107.984) (width 1) (layer "B.Cu") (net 22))
 (segment (start 109.84 108.238) (end 109.641 108.238) (width 1) (layer "B.Cu") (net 22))
 (segment (start 101.966 108.023) (end 101.99 108.047) (width 0.25) (layer "B.Cu") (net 21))
 (segment (start 101.966 102.904) (end 101.966 108.023) (width 1) (layer "B.Cu") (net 21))
 (segment (start 122.794 101.762) (end 125.125 101.762) (width 0.5) (layer "B.Cu") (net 17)))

